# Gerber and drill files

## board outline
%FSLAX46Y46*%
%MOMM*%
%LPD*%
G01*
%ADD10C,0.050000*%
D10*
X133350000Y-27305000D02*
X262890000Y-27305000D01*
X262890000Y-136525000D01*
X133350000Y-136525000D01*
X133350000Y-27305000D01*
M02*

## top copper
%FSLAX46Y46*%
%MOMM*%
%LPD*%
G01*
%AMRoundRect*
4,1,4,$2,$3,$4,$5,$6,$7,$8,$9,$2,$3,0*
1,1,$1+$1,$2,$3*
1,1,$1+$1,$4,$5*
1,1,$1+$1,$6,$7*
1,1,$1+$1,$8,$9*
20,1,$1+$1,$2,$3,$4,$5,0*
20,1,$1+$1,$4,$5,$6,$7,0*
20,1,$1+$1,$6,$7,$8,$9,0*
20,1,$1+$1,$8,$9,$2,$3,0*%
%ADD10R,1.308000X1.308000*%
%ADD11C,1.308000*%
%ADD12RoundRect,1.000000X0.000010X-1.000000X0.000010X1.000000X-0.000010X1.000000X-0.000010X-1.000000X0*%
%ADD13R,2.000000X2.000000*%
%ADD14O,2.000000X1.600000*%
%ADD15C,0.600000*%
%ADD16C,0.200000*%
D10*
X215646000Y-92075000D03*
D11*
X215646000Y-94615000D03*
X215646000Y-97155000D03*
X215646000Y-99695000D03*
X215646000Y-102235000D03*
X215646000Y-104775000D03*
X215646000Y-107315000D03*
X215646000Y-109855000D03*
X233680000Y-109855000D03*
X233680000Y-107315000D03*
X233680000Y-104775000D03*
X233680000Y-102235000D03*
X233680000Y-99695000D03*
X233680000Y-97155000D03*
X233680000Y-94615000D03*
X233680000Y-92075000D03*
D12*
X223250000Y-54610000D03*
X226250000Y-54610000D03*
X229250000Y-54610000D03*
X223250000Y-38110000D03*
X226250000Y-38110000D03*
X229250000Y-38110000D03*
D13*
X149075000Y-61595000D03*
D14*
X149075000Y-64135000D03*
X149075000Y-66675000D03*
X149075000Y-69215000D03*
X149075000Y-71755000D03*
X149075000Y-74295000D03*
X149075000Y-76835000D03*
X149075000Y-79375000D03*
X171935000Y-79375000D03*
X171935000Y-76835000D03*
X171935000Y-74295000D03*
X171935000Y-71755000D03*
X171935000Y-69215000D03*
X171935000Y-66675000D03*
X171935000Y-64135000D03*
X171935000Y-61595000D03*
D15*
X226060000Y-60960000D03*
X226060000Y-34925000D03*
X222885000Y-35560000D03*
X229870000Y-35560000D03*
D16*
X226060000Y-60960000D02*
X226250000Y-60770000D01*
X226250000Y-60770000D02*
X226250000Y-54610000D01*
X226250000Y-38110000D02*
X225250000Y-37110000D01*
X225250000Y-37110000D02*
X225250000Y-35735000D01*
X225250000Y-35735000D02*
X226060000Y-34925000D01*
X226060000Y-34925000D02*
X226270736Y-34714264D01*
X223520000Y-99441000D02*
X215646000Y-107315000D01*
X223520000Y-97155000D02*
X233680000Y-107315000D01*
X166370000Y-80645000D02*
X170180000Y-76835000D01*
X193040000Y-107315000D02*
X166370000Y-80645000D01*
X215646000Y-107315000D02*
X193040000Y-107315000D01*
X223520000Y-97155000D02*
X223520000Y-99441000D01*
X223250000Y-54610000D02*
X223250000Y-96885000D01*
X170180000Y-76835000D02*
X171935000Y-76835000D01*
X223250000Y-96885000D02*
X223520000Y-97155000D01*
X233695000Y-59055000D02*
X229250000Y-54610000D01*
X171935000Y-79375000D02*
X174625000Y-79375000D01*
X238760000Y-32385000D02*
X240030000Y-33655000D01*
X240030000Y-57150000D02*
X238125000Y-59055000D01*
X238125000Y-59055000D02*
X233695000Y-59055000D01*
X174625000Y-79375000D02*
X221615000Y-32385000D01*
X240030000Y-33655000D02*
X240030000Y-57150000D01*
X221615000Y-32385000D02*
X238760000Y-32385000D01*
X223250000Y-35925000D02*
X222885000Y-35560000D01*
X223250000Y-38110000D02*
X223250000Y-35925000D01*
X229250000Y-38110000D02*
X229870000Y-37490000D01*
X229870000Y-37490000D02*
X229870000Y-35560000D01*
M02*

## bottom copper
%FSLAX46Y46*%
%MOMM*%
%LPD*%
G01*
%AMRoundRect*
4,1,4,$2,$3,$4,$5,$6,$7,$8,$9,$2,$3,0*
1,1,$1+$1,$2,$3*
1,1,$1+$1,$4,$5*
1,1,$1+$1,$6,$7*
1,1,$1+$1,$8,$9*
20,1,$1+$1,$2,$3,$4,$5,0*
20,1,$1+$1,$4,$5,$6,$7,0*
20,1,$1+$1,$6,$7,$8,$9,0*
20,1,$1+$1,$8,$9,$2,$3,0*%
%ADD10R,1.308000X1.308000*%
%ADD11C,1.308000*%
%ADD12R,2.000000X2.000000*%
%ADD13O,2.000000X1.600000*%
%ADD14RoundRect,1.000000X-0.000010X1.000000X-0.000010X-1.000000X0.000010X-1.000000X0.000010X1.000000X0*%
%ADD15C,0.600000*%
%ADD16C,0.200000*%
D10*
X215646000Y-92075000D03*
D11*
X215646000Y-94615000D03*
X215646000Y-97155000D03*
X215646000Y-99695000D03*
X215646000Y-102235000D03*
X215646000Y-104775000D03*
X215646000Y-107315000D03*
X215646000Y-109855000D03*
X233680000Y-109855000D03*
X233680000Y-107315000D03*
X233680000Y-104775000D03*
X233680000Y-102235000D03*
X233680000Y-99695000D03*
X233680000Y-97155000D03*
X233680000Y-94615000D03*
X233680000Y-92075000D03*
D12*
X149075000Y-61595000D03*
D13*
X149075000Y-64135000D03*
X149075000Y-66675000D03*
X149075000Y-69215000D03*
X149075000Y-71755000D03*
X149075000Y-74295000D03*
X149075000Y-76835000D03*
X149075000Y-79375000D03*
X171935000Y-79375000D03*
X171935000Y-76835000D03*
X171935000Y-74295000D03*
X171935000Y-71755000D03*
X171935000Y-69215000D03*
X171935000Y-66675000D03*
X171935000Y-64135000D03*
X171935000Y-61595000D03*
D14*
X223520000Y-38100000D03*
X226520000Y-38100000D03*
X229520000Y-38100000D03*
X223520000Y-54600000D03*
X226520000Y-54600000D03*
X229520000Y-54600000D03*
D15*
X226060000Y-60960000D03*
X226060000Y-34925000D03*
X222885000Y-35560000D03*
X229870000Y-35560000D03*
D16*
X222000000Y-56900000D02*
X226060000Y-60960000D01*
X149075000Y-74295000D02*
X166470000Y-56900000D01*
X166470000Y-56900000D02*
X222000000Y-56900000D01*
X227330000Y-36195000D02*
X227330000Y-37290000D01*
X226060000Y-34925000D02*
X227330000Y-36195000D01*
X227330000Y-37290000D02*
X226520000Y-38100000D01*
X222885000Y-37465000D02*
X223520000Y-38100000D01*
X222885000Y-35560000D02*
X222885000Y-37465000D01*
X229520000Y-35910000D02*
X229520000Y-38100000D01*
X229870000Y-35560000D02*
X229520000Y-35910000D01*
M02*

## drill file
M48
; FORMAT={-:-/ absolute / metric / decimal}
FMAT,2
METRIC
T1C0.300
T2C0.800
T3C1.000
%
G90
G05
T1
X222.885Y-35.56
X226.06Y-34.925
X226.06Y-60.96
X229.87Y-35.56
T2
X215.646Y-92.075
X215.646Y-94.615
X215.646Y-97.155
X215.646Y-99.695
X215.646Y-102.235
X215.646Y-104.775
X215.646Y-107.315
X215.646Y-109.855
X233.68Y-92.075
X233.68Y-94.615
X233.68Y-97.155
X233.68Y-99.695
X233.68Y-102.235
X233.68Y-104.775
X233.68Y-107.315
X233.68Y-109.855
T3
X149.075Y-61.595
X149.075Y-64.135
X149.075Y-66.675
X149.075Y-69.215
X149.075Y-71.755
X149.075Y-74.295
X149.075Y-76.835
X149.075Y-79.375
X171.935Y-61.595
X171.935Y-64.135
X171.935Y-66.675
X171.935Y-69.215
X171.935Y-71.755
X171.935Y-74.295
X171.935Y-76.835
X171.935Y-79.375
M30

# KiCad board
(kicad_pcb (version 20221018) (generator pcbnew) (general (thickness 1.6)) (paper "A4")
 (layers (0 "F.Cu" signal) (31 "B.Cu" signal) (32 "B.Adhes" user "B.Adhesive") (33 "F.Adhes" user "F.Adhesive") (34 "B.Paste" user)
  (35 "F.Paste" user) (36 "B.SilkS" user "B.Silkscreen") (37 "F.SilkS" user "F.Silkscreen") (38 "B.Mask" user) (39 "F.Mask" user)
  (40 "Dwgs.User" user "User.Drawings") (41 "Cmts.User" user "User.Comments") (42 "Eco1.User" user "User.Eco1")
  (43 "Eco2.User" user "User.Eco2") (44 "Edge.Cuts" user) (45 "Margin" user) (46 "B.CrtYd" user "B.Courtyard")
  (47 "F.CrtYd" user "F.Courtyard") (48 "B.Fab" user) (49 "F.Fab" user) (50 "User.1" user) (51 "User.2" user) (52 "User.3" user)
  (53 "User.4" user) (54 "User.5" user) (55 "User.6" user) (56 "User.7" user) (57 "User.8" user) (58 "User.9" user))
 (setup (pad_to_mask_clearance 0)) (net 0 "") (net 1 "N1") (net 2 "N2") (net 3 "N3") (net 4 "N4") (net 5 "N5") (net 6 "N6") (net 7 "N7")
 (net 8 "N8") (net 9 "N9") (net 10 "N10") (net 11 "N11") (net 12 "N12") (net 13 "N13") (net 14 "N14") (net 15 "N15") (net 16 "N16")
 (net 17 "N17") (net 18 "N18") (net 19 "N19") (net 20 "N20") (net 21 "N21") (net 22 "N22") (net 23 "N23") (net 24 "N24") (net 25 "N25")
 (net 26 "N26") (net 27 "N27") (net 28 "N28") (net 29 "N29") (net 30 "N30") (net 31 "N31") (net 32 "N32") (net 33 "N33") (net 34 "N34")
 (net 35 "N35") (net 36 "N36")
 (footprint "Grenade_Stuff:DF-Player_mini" (layer "F.Cu") (at 224.663 100.965)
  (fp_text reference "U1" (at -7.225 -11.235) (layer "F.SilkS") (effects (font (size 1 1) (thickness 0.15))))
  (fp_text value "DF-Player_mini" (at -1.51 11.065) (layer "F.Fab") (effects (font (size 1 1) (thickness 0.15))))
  (pad "1" thru_hole rect (at -9.017 -8.89) (size 1.308 1.308) (drill 0.8) (layers "*.Cu" "*.Mask") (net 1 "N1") (solder_mask_margin 0.102))
  (pad "2" thru_hole circle (at -9.017 -6.35) (size 1.308 1.308) (drill 0.8) (layers "*.Cu" "*.Mask") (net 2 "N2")
   (solder_mask_margin 0.102))
  (pad "3" thru_hole circle (at -9.017 -3.81) (size 1.308 1.308) (drill 0.8) (layers "*.Cu" "*.Mask") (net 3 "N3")
   (solder_mask_margin 0.102))
  (pad "4" thru_hole circle (at -9.017 -1.27) (size 1.308 1.308) (drill 0.8) (layers "*.Cu" "*.Mask") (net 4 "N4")
   (solder_mask_margin 0.102))
  (pad "5" thru_hole circle (at -9.017 1.27) (size 1.308 1.308) (drill 0.8) (layers "*.Cu" "*.Mask") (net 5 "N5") (solder_mask_margin 0.102))
  (pad "6" thru_hole circle (at -9.017 3.81) (size 1.308 1.308) (drill 0.8) (layers "*.Cu" "*.Mask") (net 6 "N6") (solder_mask_margin 0.102))
  (pad "7" thru_hole circle (at -9.017 6.35) (size 1.308 1.308) (drill 0.8) (layers "*.Cu" "*.Mask") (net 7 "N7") (solder_mask_margin 0.102))
  (pad "8" thru_hole circle (at -9.017 8.89) (size 1.308 1.308) (drill 0.8) (layers "*.Cu" "*.Mask") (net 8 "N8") (solder_mask_margin 0.102))
  (pad "9" thru_hole circle (at 9.017 8.89) (size 1.308 1.308) (drill 0.8) (layers "*.Cu" "*.Mask") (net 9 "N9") (solder_mask_margin 0.102))
  (pad "10" thru_hole circle (at 9.017 6.35) (size 1.308 1.308) (drill 0.8) (layers "*.Cu" "*.Mask") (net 7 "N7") (solder_mask_margin 0.102))
  (pad "11" thru_hole circle (at 9.017 3.81) (size 1.308 1.308) (drill 0.8) (layers "*.Cu" "*.Mask") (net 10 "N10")
   (solder_mask_margin 0.102))
  (pad "12" thru_hole circle (at 9.017 1.27) (size 1.308 1.308) (drill 0.8) (layers "*.Cu" "*.Mask") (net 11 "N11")
   (solder_mask_margin 0.102))
  (pad "13" thru_hole circle (at 9.017 -1.27) (size 1.308 1.308) (drill 0.8) (layers "*.Cu" "*.Mask") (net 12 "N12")
   (solder_mask_margin 0.102))
  (pad "14" thru_hole circle (at 9.017 -3.81) (size 1.308 1.308) (drill 0.8) (layers "*.Cu" "*.Mask") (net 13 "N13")
   (solder_mask_margin 0.102))
  (pad "15" thru_hole circle (at 9.017 -6.35) (size 1.308 1.308) (drill 0.8) (layers "*.Cu" "*.Mask") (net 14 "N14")
   (solder_mask_margin 0.102))
  (pad "16" thru_hole circle (at 9.017 -8.89) (size 1.308 1.308) (drill 0.8) (layers "*.Cu" "*.Mask") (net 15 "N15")
   (solder_mask_margin 0.102)))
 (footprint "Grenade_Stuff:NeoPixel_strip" (layer "F.Cu") (at 227.06 45.72)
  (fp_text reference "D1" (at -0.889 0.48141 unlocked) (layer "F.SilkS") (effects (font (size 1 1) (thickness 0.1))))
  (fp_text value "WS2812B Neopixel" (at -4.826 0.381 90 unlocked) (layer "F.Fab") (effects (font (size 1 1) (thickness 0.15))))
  (pad "1" smd roundrect (at -3.81 8.89 90) (size 4 2) (layers "F.Cu" "F.Paste" "F.Mask") (roundrect_rratio 0.5) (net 7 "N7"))
  (pad "2" smd roundrect (at -0.81 8.89 90) (size 4 2) (layers "F.Cu" "F.Paste" "F.Mask") (roundrect_rratio 0.5) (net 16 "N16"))
  (pad "3" smd roundrect (at 2.19 8.89 90) (size 4 2) (layers "F.Cu" "F.Paste" "F.Mask") (roundrect_rratio 0.5) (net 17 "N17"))
  (pad "4" smd roundrect (at -3.81 -7.61 90) (size 4 2) (layers "F.Cu" "F.Paste" "F.Mask") (roundrect_rratio 0.5) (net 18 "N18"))
  (pad "5" smd roundrect (at -0.81 -7.61 90) (size 4 2) (layers "F.Cu" "F.Paste" "F.Mask") (roundrect_rratio 0.5) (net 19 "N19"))
  (pad "6" smd roundrect (at 2.19 -7.61 90) (size 4 2) (layers "F.Cu" "F.Paste" "F.Mask") (roundrect_rratio 0.5) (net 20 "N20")))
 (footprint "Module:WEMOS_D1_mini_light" (layer "F.Cu") (at 149.075 61.595)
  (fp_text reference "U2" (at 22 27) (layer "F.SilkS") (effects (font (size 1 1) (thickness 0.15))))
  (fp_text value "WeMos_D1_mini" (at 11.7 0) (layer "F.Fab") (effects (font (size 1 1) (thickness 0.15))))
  (pad "1" thru_hole rect (at 0 0) (size 2 2) (drill 1) (layers "*.Cu" "*.Mask") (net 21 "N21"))
  (pad "2" thru_hole oval (at 0 2.54) (size 2 1.6) (drill 1) (layers "*.Cu" "*.Mask") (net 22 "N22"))
  (pad "3" thru_hole oval (at 0 5.08) (size 2 1.6) (drill 1) (layers "*.Cu" "*.Mask") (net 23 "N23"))
  (pad "4" thru_hole oval (at 0 7.62) (size 2 1.6) (drill 1) (layers "*.Cu" "*.Mask") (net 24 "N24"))
  (pad "5" thru_hole oval (at 0 10.16) (size 2 1.6) (drill 1) (layers "*.Cu" "*.Mask") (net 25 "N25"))
  (pad "6" thru_hole oval (at 0 12.7) (size 2 1.6) (drill 1) (layers "*.Cu" "*.Mask") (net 16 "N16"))
  (pad "7" thru_hole oval (at 0 15.24) (size 2 1.6) (drill 1) (layers "*.Cu" "*.Mask") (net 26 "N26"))
  (pad "8" thru_hole oval (at 0 17.78) (size 2 1.6) (drill 1) (layers "*.Cu" "*.Mask") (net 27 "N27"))
  (pad "9" thru_hole oval (at 22.86 17.78) (size 2 1.6) (drill 1) (layers "*.Cu" "*.Mask") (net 17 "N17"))
  (pad "10" thru_hole oval (at 22.86 15.24) (size 2 1.6) (drill 1) (layers "*.Cu" "*.Mask") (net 7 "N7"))
  (pad "11" thru_hole oval (at 22.86 12.7) (size 2 1.6) (drill 1) (layers "*.Cu" "*.Mask") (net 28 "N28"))
  (pad "12" thru_hole oval (at 22.86 10.16) (size 2 1.6) (drill 1) (layers "*.Cu" "*.Mask") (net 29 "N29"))
  (pad "13" thru_hole oval (at 22.86 7.62) (size 2 1.6) (drill 1) (layers "*.Cu" "*.Mask") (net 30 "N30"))
  (pad "14" thru_hole oval (at 22.86 5.08) (size 2 1.6) (drill 1) (layers "*.Cu" "*.Mask") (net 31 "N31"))
  (pad "15" thru_hole oval (at 22.86 2.54) (size 2 1.6) (drill 1) (layers "*.Cu" "*.Mask") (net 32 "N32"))
  (pad "16" thru_hole oval (at 22.86 0) (size 2 1.6) (drill 1) (layers "*.Cu" "*.Mask") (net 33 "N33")))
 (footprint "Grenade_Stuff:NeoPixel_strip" (layer "B.Cu") (at 227.33 46.99)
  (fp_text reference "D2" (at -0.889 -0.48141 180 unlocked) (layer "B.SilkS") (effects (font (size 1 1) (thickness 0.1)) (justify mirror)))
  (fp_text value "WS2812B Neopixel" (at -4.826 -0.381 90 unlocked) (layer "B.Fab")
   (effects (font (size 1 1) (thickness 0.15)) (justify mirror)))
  (pad "1" smd roundrect (at -3.81 -8.89 270) (size 4 2) (layers "B.Cu" "B.Paste" "B.Mask") (roundrect_rratio 0.5) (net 18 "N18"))
  (pad "2" smd roundrect (at -0.81 -8.89 270) (size 4 2) (layers "B.Cu" "B.Paste" "B.Mask") (roundrect_rratio 0.5) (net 19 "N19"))
  (pad "3" smd roundrect (at 2.19 -8.89 270) (size 4 2) (layers "B.Cu" "B.Paste" "B.Mask") (roundrect_rratio 0.5) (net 20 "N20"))
  (pad "4" smd roundrect (at -3.81 7.61 270) (size 4 2) (layers "B.Cu" "B.Paste" "B.Mask") (roundrect_rratio 0.5) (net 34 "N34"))
  (pad "5" smd roundrect (at -0.81 7.61 270) (size 4 2) (layers "B.Cu" "B.Paste" "B.Mask") (roundrect_rratio 0.5) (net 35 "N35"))
  (pad "6" smd roundrect (at 2.19 7.61 270) (size 4 2) (layers "B.Cu" "B.Paste" "B.Mask") (roundrect_rratio 0.5) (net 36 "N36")))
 (gr_rect (start 133.35 27.305) (end 262.89 136.525) (stroke (width 0.05) (type default)) (fill none) (layer "Edge.Cuts"))
 (segment (start 226.06 60.96) (end 226.25 60.77) (width 0.2) (layer "F.Cu") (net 16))
 (segment (start 226.25 60.77) (end 226.25 54.61) (width 0.2) (layer "F.Cu") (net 16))
 (via (at 226.06 60.96) (size 0.6) (drill 0.3) (layers "F.Cu" "B.Cu") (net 16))
 (segment (start 222 56.9) (end 226.06 60.96) (width 0.2) (layer "B.Cu") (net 16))
 (segment (start 149.075 74.295) (end 166.47 56.9) (width 0.2) (layer "B.Cu") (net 16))
 (segment (start 166.47 56.9) (end 222 56.9) (width 0.2) (layer "B.Cu") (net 16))
 (segment (start 226.25 38.11) (end 225.25 37.11) (width 0.2) (layer "F.Cu") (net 19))
 (segment (start 225.25 37.11) (end 225.25 35.735) (width 0.2) (layer "F.Cu") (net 19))
 (segment (start 225.25 35.735) (end 226.06 34.925) (width 0.2) (layer "F.Cu") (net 19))
 (segment (start 226.06 34.925) (end 226.270736 34.714264) (width 0.2) (layer "F.Cu") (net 19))
 (via (at 226.06 34.925) (size 0.6) (drill 0.3) (layers "F.Cu" "B.Cu") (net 19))
 (segment (start 227.33 36.195) (end 227.33 37.29) (width 0.2) (layer "B.Cu") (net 19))
 (segment (start 226.06 34.925) (end 227.33 36.195) (width 0.2) (layer "B.Cu") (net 19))
 (segment (start 227.33 37.29) (end 226.52 38.1) (width 0.2) (layer "B.Cu") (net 19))
 (segment (start 223.52 99.441) (end 215.646 107.315) (width 0.2) (layer "F.Cu") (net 7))
 (segment (start 223.52 97.155) (end 233.68 107.315) (width 0.2) (layer "F.Cu") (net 7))
 (segment (start 166.37 80.645) (end 170.18 76.835) (width 0.2) (layer "F.Cu") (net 7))
 (segment (start 193.04 107.315) (end 166.37 80.645) (width 0.2) (layer "F.Cu") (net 7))
 (segment (start 215.646 107.315) (end 193.04 107.315) (width 0.2) (layer "F.Cu") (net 7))
 (segment (start 223.52 97.155) (end 223.52 99.441) (width 0.2) (layer "F.Cu") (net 7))
 (segment (start 223.25 54.61) (end 223.25 96.885) (width 0.2) (layer "F.Cu") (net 7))
 (segment (start 170.18 76.835) (end 171.935 76.835) (width 0.2) (layer "F.Cu") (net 7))
 (segment (start 223.25 96.885) (end 223.52 97.155) (width 0.2) (layer "F.Cu") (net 7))
 (segment (start 233.695 59.055) (end 229.25 54.61) (width 0.2) (layer "F.Cu") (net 17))
 (segment (start 171.935 79.375) (end 174.625 79.375) (width 0.2) (layer "F.Cu") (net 17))
 (segment (start 238.76 32.385) (end 240.03 33.655) (width 0.2) (layer "F.Cu") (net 17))
 (segment (start 240.03 57.15) (end 238.125 59.055) (width 0.2) (layer "F.Cu") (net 17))
 (segment (start 238.125 59.055) (end 233.695 59.055) (width 0.2) (layer "F.Cu") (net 17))
 (segment (start 174.625 79.375) (end 221.615 32.385) (width 0.2) (layer "F.Cu") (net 17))
 (segment (start 240.03 33.655) (end 240.03 57.15) (width 0.2) (layer "F.Cu") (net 17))
 (segment (start 221.615 32.385) (end 238.76 32.385) (width 0.2) (layer "F.Cu") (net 17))
 (segment (start 223.25 35.925) (end 222.885 35.56) (width 0.2) (layer "F.Cu") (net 18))
 (segment (start 223.25 38.11) (end 223.25 35.925) (width 0.2) (layer "F.Cu") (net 18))
 (via (at 222.885 35.56) (size 0.6) (drill 0.3) (layers "F.Cu" "B.Cu") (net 18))
 (segment (start 222.885 37.465) (end 223.52 38.1) (width 0.2) (layer "B.Cu") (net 18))
 (segment (start 222.885 35.56) (end 222.885 37.465) (width 0.2) (layer "B.Cu") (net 18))
 (segment (start 229.25 38.11) (end 229.87 37.49) (width 0.2) (layer "F.Cu") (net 20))
 (segment (start 229.87 37.49) (end 229.87 35.56) (width 0.2) (layer "F.Cu") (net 20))
 (via (at 229.87 35.56) (size 0.6) (drill 0.3) (layers "F.Cu" "B.Cu") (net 20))
 (segment (start 229.52 35.91) (end 229.52 38.1) (width 0.2) (layer "B.Cu") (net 20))
 (segment (start 229.87 35.56) (end 229.52 35.91) (width 0.2) (layer "B.Cu") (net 20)))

